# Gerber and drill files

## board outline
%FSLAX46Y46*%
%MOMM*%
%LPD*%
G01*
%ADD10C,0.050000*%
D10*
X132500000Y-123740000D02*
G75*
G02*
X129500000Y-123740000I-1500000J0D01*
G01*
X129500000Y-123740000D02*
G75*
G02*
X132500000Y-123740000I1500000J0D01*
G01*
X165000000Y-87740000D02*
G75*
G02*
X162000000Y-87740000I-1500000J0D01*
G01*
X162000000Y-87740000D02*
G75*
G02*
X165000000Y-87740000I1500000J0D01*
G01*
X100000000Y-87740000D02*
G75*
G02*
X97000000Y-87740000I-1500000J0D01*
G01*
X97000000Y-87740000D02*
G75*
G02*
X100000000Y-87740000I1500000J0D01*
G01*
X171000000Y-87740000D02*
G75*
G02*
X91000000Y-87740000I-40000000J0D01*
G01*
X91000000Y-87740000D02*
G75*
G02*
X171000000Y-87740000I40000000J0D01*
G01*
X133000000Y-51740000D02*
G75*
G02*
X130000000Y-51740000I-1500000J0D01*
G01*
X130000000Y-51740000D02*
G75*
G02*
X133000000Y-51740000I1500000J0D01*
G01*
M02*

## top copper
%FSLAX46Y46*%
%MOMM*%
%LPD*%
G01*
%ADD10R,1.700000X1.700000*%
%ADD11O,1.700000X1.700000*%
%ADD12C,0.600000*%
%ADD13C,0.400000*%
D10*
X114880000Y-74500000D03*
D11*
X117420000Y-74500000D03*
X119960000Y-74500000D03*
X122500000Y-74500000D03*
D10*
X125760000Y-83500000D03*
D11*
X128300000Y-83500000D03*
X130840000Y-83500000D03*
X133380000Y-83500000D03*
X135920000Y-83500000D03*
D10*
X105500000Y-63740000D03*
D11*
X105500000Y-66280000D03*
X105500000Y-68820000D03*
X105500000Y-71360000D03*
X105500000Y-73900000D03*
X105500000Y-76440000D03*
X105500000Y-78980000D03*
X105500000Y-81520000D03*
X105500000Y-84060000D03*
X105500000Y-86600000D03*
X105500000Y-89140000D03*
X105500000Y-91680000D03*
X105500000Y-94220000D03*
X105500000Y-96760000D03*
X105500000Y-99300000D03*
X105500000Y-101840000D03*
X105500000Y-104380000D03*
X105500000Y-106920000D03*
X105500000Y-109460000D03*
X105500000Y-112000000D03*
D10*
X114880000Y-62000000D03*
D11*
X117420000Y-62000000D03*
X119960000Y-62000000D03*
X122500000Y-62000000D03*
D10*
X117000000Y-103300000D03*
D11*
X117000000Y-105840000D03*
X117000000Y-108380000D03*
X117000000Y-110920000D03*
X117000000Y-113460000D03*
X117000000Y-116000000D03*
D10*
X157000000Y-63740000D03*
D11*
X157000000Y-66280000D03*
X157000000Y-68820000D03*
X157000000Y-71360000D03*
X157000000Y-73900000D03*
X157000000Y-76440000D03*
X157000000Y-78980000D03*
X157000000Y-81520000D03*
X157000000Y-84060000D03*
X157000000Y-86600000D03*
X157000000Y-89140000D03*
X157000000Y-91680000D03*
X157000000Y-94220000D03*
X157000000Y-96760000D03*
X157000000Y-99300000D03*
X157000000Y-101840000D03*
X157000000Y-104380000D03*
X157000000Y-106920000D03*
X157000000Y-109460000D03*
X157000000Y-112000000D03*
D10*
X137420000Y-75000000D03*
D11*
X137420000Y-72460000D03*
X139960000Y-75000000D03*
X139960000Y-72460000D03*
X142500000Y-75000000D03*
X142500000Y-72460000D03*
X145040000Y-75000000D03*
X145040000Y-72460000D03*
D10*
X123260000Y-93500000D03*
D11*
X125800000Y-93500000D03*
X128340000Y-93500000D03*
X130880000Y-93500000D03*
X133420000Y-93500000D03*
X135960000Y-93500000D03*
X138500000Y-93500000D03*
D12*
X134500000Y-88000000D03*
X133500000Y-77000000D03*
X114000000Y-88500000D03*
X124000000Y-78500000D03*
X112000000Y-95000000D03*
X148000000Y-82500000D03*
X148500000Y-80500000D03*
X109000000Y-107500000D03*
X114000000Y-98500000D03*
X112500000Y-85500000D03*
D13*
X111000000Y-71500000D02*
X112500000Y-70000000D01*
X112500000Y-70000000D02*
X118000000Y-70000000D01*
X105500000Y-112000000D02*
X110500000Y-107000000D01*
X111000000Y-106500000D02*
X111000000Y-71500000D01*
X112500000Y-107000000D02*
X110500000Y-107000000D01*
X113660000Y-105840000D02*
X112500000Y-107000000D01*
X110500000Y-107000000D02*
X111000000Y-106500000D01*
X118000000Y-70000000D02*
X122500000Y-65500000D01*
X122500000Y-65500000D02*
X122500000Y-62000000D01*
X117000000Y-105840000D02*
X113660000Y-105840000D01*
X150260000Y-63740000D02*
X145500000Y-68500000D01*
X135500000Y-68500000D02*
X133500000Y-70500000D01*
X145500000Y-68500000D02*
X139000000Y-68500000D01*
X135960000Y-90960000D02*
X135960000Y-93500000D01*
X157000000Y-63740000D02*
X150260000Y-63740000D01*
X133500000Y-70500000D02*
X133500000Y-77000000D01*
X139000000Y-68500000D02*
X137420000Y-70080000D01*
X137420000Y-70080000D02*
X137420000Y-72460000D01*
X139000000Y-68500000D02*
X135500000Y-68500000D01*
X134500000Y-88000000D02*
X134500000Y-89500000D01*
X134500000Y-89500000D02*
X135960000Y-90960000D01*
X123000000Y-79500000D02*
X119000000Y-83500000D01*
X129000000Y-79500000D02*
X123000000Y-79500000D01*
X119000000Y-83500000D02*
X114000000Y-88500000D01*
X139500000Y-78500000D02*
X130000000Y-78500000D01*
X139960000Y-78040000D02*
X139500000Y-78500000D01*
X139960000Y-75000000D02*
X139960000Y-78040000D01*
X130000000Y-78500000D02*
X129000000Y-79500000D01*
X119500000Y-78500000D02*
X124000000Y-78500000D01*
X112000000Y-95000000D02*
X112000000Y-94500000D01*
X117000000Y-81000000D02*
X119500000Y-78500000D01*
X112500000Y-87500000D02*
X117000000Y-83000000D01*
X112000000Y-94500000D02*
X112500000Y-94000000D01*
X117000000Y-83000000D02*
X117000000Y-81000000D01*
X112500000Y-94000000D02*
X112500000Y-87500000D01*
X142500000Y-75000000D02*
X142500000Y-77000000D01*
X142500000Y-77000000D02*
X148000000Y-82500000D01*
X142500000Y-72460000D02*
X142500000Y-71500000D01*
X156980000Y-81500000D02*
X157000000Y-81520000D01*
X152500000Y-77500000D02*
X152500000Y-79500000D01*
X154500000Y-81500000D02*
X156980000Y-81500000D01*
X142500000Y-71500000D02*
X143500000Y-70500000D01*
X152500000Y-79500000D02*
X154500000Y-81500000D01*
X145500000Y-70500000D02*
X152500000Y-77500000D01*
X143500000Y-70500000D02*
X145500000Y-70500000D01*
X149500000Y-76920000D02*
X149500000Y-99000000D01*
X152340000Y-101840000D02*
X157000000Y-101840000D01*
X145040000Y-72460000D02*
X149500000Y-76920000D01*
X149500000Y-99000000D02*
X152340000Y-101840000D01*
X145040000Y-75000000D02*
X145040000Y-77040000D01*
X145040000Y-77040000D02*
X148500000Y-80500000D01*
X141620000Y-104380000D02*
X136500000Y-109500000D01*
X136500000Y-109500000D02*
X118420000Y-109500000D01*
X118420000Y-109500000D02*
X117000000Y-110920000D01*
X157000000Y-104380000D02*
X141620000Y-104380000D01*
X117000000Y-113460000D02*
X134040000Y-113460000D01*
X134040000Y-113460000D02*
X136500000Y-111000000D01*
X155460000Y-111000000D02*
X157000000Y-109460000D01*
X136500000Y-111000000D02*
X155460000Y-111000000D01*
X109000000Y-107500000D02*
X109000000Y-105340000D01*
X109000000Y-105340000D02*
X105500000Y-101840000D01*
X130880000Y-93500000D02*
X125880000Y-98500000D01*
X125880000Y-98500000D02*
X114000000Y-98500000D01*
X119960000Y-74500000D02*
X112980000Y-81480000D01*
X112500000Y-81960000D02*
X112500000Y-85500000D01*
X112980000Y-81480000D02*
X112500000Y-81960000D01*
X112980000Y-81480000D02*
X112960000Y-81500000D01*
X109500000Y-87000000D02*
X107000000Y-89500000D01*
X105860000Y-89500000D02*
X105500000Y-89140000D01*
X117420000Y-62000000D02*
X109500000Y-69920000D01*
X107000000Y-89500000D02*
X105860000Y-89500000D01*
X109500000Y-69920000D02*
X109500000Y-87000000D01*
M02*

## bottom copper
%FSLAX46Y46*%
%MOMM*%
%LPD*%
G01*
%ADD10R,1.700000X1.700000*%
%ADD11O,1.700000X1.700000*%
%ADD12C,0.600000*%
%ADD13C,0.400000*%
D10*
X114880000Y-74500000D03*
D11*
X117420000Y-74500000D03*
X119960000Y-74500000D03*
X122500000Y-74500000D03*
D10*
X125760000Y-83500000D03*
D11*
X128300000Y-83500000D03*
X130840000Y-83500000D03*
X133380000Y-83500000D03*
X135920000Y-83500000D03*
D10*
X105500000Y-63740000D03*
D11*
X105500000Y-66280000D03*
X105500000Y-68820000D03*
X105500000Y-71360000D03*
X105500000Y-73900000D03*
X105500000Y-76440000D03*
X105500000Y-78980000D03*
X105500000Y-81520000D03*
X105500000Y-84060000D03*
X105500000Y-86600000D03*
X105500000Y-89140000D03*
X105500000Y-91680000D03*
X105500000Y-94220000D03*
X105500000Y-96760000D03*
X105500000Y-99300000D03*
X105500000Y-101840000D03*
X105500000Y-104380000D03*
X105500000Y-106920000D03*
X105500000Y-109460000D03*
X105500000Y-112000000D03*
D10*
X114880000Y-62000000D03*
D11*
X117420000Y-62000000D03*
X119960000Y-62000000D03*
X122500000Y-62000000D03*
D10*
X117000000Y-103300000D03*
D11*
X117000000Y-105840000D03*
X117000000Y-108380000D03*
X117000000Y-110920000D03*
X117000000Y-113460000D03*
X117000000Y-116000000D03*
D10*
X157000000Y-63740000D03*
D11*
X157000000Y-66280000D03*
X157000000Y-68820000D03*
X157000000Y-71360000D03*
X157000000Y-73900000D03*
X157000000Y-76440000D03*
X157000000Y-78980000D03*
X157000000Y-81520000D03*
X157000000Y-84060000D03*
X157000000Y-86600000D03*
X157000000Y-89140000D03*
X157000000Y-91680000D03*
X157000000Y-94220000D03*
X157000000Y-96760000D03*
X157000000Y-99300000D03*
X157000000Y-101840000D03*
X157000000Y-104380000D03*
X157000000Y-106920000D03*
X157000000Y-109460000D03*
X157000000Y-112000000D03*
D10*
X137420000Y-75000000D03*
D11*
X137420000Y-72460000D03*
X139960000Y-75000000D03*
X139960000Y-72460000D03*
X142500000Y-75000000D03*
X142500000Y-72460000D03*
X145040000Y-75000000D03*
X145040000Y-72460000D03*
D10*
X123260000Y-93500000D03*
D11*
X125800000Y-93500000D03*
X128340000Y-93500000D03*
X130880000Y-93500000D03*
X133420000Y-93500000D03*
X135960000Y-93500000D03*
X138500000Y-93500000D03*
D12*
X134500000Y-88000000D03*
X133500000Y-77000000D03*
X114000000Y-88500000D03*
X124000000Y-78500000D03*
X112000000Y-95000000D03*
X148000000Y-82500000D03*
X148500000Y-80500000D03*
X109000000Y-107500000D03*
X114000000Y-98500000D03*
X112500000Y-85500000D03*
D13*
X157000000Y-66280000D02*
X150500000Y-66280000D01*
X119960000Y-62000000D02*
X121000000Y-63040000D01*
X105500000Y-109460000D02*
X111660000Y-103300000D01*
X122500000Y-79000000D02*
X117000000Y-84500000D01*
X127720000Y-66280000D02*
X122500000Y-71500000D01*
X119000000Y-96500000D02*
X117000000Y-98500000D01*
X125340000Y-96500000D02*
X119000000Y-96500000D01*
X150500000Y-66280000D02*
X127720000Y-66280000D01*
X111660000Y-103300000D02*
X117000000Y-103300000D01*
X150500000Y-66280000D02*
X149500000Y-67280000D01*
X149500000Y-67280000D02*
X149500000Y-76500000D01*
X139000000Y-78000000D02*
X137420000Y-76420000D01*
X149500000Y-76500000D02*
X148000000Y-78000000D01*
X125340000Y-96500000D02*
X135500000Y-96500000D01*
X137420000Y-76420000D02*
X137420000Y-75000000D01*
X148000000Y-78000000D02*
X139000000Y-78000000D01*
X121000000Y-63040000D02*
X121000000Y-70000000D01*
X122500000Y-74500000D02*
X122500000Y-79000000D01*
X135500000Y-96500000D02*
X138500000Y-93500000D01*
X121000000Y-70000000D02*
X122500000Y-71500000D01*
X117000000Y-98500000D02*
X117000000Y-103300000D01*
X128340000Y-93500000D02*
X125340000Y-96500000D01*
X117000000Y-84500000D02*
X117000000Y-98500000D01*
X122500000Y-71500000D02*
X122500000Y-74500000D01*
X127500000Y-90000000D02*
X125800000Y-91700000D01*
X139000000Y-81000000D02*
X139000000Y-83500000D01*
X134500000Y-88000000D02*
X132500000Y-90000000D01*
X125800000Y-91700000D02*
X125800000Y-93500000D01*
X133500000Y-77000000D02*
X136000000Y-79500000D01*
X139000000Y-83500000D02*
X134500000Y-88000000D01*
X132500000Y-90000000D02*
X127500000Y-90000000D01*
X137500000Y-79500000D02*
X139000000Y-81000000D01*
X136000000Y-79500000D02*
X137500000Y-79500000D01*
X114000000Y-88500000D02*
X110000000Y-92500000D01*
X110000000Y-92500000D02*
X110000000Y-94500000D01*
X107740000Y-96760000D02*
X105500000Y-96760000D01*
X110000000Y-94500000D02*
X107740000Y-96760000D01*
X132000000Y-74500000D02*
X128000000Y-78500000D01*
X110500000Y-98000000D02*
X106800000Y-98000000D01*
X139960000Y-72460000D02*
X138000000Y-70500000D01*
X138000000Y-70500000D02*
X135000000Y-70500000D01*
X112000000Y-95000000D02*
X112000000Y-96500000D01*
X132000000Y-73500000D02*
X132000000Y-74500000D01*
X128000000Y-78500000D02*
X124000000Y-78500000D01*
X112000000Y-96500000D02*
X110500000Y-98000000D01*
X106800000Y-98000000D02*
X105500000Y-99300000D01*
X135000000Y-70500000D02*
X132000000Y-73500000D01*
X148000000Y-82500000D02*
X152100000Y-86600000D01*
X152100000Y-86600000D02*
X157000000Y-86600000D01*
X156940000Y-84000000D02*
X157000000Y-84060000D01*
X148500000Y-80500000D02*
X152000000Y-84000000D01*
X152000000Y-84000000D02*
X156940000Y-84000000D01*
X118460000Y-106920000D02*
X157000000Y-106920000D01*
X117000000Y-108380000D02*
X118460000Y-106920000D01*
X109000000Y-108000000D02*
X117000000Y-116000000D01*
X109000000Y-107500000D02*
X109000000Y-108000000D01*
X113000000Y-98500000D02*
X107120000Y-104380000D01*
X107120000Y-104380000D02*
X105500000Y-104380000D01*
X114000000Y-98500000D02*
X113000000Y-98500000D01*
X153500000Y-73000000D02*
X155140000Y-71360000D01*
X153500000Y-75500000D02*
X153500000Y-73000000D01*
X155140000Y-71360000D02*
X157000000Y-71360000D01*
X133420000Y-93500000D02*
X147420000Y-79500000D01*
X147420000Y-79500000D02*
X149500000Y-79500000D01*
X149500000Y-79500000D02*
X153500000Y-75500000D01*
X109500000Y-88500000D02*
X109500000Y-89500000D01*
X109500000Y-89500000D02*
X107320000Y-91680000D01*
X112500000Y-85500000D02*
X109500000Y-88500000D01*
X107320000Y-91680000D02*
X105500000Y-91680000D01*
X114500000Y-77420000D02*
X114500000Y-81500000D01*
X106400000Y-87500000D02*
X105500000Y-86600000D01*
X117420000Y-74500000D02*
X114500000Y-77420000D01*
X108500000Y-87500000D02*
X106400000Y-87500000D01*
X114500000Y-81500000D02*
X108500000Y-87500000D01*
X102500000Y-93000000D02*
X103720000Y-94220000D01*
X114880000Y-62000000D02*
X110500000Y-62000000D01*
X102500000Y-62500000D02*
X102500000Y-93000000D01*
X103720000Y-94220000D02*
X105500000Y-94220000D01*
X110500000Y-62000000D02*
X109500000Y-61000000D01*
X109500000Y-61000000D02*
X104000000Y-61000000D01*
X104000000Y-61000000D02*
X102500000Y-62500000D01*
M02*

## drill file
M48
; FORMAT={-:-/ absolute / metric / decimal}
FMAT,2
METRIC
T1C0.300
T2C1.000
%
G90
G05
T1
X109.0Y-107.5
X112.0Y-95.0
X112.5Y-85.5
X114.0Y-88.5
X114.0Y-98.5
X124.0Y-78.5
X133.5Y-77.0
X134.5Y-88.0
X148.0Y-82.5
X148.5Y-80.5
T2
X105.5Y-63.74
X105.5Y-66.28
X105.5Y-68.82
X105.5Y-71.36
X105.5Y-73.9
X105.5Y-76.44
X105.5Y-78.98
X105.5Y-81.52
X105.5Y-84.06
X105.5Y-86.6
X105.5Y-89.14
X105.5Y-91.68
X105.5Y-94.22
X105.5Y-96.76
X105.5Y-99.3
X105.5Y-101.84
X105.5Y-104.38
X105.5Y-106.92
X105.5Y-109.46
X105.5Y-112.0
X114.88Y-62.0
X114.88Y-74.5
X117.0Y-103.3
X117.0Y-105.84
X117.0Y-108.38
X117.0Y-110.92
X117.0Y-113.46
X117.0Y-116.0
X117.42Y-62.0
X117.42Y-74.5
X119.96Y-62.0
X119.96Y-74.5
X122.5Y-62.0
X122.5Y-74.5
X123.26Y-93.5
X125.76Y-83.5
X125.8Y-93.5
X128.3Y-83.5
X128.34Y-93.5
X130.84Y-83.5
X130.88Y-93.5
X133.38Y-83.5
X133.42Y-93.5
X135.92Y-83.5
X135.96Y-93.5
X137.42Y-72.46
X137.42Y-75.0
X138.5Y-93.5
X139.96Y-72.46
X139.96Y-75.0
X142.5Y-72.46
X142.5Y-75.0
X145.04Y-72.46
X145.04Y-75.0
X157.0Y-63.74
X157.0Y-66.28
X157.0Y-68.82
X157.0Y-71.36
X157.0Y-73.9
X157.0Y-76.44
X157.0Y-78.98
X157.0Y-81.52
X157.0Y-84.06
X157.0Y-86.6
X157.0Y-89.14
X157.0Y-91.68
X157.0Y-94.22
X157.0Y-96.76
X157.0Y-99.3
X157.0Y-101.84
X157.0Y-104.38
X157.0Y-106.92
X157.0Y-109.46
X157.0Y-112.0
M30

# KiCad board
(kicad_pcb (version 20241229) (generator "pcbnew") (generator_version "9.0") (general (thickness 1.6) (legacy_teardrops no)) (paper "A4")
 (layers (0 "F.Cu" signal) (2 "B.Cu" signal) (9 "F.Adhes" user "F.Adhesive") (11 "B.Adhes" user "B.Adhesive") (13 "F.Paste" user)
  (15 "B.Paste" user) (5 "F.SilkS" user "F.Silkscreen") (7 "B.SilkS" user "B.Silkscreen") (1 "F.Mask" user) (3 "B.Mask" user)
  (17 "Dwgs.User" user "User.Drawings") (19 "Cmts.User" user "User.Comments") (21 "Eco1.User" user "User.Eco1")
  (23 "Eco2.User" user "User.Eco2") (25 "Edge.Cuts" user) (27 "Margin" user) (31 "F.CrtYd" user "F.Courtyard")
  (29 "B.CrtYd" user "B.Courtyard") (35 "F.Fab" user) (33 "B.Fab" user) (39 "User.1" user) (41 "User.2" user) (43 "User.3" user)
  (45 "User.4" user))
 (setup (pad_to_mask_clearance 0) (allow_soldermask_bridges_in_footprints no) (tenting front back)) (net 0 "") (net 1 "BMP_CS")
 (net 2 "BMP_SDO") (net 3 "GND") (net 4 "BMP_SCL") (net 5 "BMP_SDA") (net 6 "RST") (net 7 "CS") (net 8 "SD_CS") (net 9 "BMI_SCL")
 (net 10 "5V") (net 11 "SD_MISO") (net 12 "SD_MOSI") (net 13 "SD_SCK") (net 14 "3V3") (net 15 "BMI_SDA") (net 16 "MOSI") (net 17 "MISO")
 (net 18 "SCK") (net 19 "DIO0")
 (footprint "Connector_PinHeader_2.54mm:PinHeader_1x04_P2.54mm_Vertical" (layer "F.Cu") (at 114.88 74.5 90)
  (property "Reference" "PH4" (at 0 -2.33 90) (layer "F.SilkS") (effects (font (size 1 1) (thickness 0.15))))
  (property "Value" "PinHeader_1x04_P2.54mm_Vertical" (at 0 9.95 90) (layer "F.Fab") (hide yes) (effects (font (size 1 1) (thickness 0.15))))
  (pad "1" thru_hole rect (at 0 0 90) (size 1.7 1.7) (drill 1) (layers "*.Cu" "*.Mask") (remove_unused_layers no))
  (pad "2" thru_hole oval (at 0 2.54 90) (size 1.7 1.7) (drill 1) (layers "*.Cu" "*.Mask") (remove_unused_layers no) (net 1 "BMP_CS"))
  (pad "3" thru_hole oval (at 0 5.08 90) (size 1.7 1.7) (drill 1) (layers "*.Cu" "*.Mask") (remove_unused_layers no) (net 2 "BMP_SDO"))
  (pad "4" thru_hole oval (at 0 7.62 90) (size 1.7 1.7) (drill 1) (layers "*.Cu" "*.Mask") (remove_unused_layers no) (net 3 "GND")))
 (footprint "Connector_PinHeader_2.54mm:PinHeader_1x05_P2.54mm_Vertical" (layer "F.Cu") (at 125.76 83.5 90)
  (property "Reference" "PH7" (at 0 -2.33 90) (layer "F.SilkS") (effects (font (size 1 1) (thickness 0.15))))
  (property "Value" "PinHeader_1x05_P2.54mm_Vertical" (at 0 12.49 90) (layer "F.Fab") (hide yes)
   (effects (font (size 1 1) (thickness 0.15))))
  (pad "1" thru_hole rect (at 0 0 90) (size 1.7 1.7) (drill 1) (layers "*.Cu" "*.Mask") (remove_unused_layers no))
  (pad "2" thru_hole oval (at 0 2.54 90) (size 1.7 1.7) (drill 1) (layers "*.Cu" "*.Mask") (remove_unused_layers no))
  (pad "3" thru_hole oval (at 0 5.08 90) (size 1.7 1.7) (drill 1) (layers "*.Cu" "*.Mask") (remove_unused_layers no))
  (pad "4" thru_hole oval (at 0 7.62 90) (size 1.7 1.7) (drill 1) (layers "*.Cu" "*.Mask") (remove_unused_layers no))
  (pad "5" thru_hole oval (at 0 10.16 90) (size 1.7 1.7) (drill 1) (layers "*.Cu" "*.Mask") (remove_unused_layers no)))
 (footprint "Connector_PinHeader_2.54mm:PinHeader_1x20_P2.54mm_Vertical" (layer "F.Cu") (at 105.5 63.74)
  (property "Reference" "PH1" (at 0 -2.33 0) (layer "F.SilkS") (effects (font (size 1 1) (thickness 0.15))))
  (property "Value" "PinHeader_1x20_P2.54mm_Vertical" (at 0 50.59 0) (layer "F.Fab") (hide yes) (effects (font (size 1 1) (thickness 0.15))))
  (pad "1" thru_hole rect (at 0 0) (size 1.7 1.7) (drill 1) (layers "*.Cu" "*.Mask") (remove_unused_layers no))
  (pad "2" thru_hole oval (at 0 2.54) (size 1.7 1.7) (drill 1) (layers "*.Cu" "*.Mask") (remove_unused_layers no))
  (pad "3" thru_hole oval (at 0 5.08) (size 1.7 1.7) (drill 1) (layers "*.Cu" "*.Mask") (remove_unused_layers no))
  (pad "4" thru_hole oval (at 0 7.62) (size 1.7 1.7) (drill 1) (layers "*.Cu" "*.Mask") (remove_unused_layers no))
  (pad "5" thru_hole oval (at 0 10.16) (size 1.7 1.7) (drill 1) (layers "*.Cu" "*.Mask") (remove_unused_layers no))
  (pad "6" thru_hole oval (at 0 12.7) (size 1.7 1.7) (drill 1) (layers "*.Cu" "*.Mask") (remove_unused_layers no))
  (pad "7" thru_hole oval (at 0 15.24) (size 1.7 1.7) (drill 1) (layers "*.Cu" "*.Mask") (remove_unused_layers no))
  (pad "8" thru_hole oval (at 0 17.78) (size 1.7 1.7) (drill 1) (layers "*.Cu" "*.Mask") (remove_unused_layers no))
  (pad "9" thru_hole oval (at 0 20.32) (size 1.7 1.7) (drill 1) (layers "*.Cu" "*.Mask") (remove_unused_layers no))
  (pad "10" thru_hole oval (at 0 22.86) (size 1.7 1.7) (drill 1) (layers "*.Cu" "*.Mask") (remove_unused_layers no) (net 1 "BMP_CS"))
  (pad "11" thru_hole oval (at 0 25.4) (size 1.7 1.7) (drill 1) (layers "*.Cu" "*.Mask") (remove_unused_layers no) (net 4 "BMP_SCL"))
  (pad "12" thru_hole oval (at 0 27.94) (size 1.7 1.7) (drill 1) (layers "*.Cu" "*.Mask") (remove_unused_layers no) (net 2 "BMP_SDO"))
  (pad "13" thru_hole oval (at 0 30.48) (size 1.7 1.7) (drill 1) (layers "*.Cu" "*.Mask") (remove_unused_layers no) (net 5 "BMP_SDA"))
  (pad "14" thru_hole oval (at 0 33.02) (size 1.7 1.7) (drill 1) (layers "*.Cu" "*.Mask") (remove_unused_layers no) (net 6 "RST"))
  (pad "15" thru_hole oval (at 0 35.56) (size 1.7 1.7) (drill 1) (layers "*.Cu" "*.Mask") (remove_unused_layers no) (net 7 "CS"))
  (pad "16" thru_hole oval (at 0 38.1) (size 1.7 1.7) (drill 1) (layers "*.Cu" "*.Mask") (remove_unused_layers no) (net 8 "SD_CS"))
  (pad "17" thru_hole oval (at 0 40.64) (size 1.7 1.7) (drill 1) (layers "*.Cu" "*.Mask") (remove_unused_layers no) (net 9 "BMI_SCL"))
  (pad "18" thru_hole oval (at 0 43.18) (size 1.7 1.7) (drill 1) (layers "*.Cu" "*.Mask") (remove_unused_layers no))
  (pad "19" thru_hole oval (at 0 45.72) (size 1.7 1.7) (drill 1) (layers "*.Cu" "*.Mask") (remove_unused_layers no) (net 3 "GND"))
  (pad "20" thru_hole oval (at 0 48.26) (size 1.7 1.7) (drill 1) (layers "*.Cu" "*.Mask") (remove_unused_layers no) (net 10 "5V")))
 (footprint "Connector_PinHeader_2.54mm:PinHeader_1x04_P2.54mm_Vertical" (layer "F.Cu") (at 114.88 62 90)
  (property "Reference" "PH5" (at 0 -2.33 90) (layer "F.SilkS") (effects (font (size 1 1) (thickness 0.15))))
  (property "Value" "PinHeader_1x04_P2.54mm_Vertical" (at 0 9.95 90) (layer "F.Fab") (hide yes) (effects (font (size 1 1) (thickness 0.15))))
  (pad "1" thru_hole rect (at 0 0 90) (size 1.7 1.7) (drill 1) (layers "*.Cu" "*.Mask") (remove_unused_layers no) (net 5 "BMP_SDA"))
  (pad "2" thru_hole oval (at 0 2.54 90) (size 1.7 1.7) (drill 1) (layers "*.Cu" "*.Mask") (remove_unused_layers no) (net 4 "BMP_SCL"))
  (pad "3" thru_hole oval (at 0 5.08 90) (size 1.7 1.7) (drill 1) (layers "*.Cu" "*.Mask") (remove_unused_layers no) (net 3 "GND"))
  (pad "4" thru_hole oval (at 0 7.62 90) (size 1.7 1.7) (drill 1) (layers "*.Cu" "*.Mask") (remove_unused_layers no) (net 10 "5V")))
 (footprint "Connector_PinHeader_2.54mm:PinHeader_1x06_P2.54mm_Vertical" (layer "F.Cu") (at 117 103.3)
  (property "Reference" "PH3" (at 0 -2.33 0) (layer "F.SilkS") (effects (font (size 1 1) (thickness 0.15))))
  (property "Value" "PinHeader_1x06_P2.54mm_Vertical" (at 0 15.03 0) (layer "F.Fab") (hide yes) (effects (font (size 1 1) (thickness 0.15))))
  (pad "1" thru_hole rect (at 0 0) (size 1.7 1.7) (drill 1) (layers "*.Cu" "*.Mask") (remove_unused_layers no) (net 3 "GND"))
  (pad "2" thru_hole oval (at 0 2.54) (size 1.7 1.7) (drill 1) (layers "*.Cu" "*.Mask") (remove_unused_layers no) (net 10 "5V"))
  (pad "3" thru_hole oval (at 0 5.08) (size 1.7 1.7) (drill 1) (layers "*.Cu" "*.Mask") (remove_unused_layers no) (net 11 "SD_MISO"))
  (pad "4" thru_hole oval (at 0 7.62) (size 1.7 1.7) (drill 1) (layers "*.Cu" "*.Mask") (remove_unused_layers no) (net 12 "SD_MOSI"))
  (pad "5" thru_hole oval (at 0 10.16) (size 1.7 1.7) (drill 1) (layers "*.Cu" "*.Mask") (remove_unused_layers no) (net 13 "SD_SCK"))
  (pad "6" thru_hole oval (at 0 12.7) (size 1.7 1.7) (drill 1) (layers "*.Cu" "*.Mask") (remove_unused_layers no) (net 8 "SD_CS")))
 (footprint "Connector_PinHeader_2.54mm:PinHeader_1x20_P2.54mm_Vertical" (layer "F.Cu") (at 157 63.74)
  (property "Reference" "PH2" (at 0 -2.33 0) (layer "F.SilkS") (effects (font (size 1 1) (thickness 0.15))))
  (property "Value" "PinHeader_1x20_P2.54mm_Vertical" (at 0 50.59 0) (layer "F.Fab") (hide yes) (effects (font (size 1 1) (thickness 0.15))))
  (pad "1" thru_hole rect (at 0 0) (size 1.7 1.7) (drill 1) (layers "*.Cu" "*.Mask") (remove_unused_layers no) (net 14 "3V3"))
  (pad "2" thru_hole oval (at 0 2.54) (size 1.7 1.7) (drill 1) (layers "*.Cu" "*.Mask") (remove_unused_layers no) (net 3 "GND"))
  (pad "3" thru_hole oval (at 0 5.08) (size 1.7 1.7) (drill 1) (layers "*.Cu" "*.Mask") (remove_unused_layers no))
  (pad "4" thru_hole oval (at 0 7.62) (size 1.7 1.7) (drill 1) (layers "*.Cu" "*.Mask") (remove_unused_layers no) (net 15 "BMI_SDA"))
  (pad "5" thru_hole oval (at 0 10.16) (size 1.7 1.7) (drill 1) (layers "*.Cu" "*.Mask") (remove_unused_layers no))
  (pad "6" thru_hole oval (at 0 12.7) (size 1.7 1.7) (drill 1) (layers "*.Cu" "*.Mask") (remove_unused_layers no))
  (pad "7" thru_hole oval (at 0 15.24) (size 1.7 1.7) (drill 1) (layers "*.Cu" "*.Mask") (remove_unused_layers no))
  (pad "8" thru_hole oval (at 0 17.78) (size 1.7 1.7) (drill 1) (layers "*.Cu" "*.Mask") (remove_unused_layers no) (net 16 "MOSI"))
  (pad "9" thru_hole oval (at 0 20.32) (size 1.7 1.7) (drill 1) (layers "*.Cu" "*.Mask") (remove_unused_layers no) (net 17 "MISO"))
  (pad "10" thru_hole oval (at 0 22.86) (size 1.7 1.7) (drill 1) (layers "*.Cu" "*.Mask") (remove_unused_layers no) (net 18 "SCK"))
  (pad "11" thru_hole oval (at 0 25.4) (size 1.7 1.7) (drill 1) (layers "*.Cu" "*.Mask") (remove_unused_layers no))
  (pad "12" thru_hole oval (at 0 27.94) (size 1.7 1.7) (drill 1) (layers "*.Cu" "*.Mask") (remove_unused_layers no))
  (pad "13" thru_hole oval (at 0 30.48) (size 1.7 1.7) (drill 1) (layers "*.Cu" "*.Mask") (remove_unused_layers no))
  (pad "14" thru_hole oval (at 0 33.02) (size 1.7 1.7) (drill 1) (layers "*.Cu" "*.Mask") (remove_unused_layers no))
  (pad "15" thru_hole oval (at 0 35.56) (size 1.7 1.7) (drill 1) (layers "*.Cu" "*.Mask") (remove_unused_layers no))
  (pad "16" thru_hole oval (at 0 38.1) (size 1.7 1.7) (drill 1) (layers "*.Cu" "*.Mask") (remove_unused_layers no) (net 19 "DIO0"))
  (pad "17" thru_hole oval (at 0 40.64) (size 1.7 1.7) (drill 1) (layers "*.Cu" "*.Mask") (remove_unused_layers no) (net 12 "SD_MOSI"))
  (pad "18" thru_hole oval (at 0 43.18) (size 1.7 1.7) (drill 1) (layers "*.Cu" "*.Mask") (remove_unused_layers no) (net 11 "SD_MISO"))
  (pad "19" thru_hole oval (at 0 45.72) (size 1.7 1.7) (drill 1) (layers "*.Cu" "*.Mask") (remove_unused_layers no) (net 13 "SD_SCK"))
  (pad "20" thru_hole oval (at 0 48.26) (size 1.7 1.7) (drill 1) (layers "*.Cu" "*.Mask") (remove_unused_layers no)))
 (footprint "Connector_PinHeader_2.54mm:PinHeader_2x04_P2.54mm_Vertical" (layer "F.Cu") (at 137.42 75 90)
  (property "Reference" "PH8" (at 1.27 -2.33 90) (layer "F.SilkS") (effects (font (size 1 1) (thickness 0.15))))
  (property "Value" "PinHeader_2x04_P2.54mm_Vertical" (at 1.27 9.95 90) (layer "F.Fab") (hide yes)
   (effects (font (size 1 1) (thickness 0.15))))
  (pad "1" thru_hole rect (at 0 0 90) (size 1.7 1.7) (drill 1) (layers "*.Cu" "*.Mask") (remove_unused_layers no) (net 3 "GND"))
  (pad "2" thru_hole oval (at 2.54 0 90) (size 1.7 1.7) (drill 1) (layers "*.Cu" "*.Mask") (remove_unused_layers no) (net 14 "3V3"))
  (pad "3" thru_hole oval (at 0 2.54 90) (size 1.7 1.7) (drill 1) (layers "*.Cu" "*.Mask") (remove_unused_layers no) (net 6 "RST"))
  (pad "4" thru_hole oval (at 2.54 2.54 90) (size 1.7 1.7) (drill 1) (layers "*.Cu" "*.Mask") (remove_unused_layers no) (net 7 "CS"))
  (pad "5" thru_hole oval (at 0 5.08 90) (size 1.7 1.7) (drill 1) (layers "*.Cu" "*.Mask") (remove_unused_layers no) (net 18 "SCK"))
  (pad "6" thru_hole oval (at 2.54 5.08 90) (size 1.7 1.7) (drill 1) (layers "*.Cu" "*.Mask") (remove_unused_layers no) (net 16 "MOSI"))
  (pad "7" thru_hole oval (at 0 7.62 90) (size 1.7 1.7) (drill 1) (layers "*.Cu" "*.Mask") (remove_unused_layers no) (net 17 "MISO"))
  (pad "8" thru_hole oval (at 2.54 7.62 90) (size 1.7 1.7) (drill 1) (layers "*.Cu" "*.Mask") (remove_unused_layers no) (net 19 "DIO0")))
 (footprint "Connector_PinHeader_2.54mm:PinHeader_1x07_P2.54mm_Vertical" (layer "F.Cu") (at 123.26 93.5 90)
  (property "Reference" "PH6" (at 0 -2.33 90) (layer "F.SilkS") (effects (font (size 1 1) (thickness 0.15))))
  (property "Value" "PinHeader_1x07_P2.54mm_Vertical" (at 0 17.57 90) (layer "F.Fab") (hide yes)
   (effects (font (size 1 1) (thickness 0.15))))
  (pad "1" thru_hole rect (at 0 0 90) (size 1.7 1.7) (drill 1) (layers "*.Cu" "*.Mask") (remove_unused_layers no))
  (pad "2" thru_hole oval (at 0 2.54 90) (size 1.7 1.7) (drill 1) (layers "*.Cu" "*.Mask") (remove_unused_layers no) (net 14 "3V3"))
  (pad "3" thru_hole oval (at 0 5.08 90) (size 1.7 1.7) (drill 1) (layers "*.Cu" "*.Mask") (remove_unused_layers no) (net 3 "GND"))
  (pad "4" thru_hole oval (at 0 7.62 90) (size 1.7 1.7) (drill 1) (layers "*.Cu" "*.Mask") (remove_unused_layers no) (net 9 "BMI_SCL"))
  (pad "5" thru_hole oval (at 0 10.16 90) (size 1.7 1.7) (drill 1) (layers "*.Cu" "*.Mask") (remove_unused_layers no) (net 15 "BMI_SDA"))
  (pad "6" thru_hole oval (at 0 12.7 90) (size 1.7 1.7) (drill 1) (layers "*.Cu" "*.Mask") (remove_unused_layers no) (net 14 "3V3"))
  (pad "7" thru_hole oval (at 0 15.24 90) (size 1.7 1.7) (drill 1) (layers "*.Cu" "*.Mask") (remove_unused_layers no) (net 3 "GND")))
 (gr_circle (center 131 123.74) (end 132.5 123.74) (stroke (width 0.05) (type default)) (fill no) (layer "Edge.Cuts"))
 (gr_circle (center 163.5 87.74) (end 165 87.74) (stroke (width 0.05) (type default)) (fill no) (layer "Edge.Cuts"))
 (gr_circle (center 98.5 87.74) (end 100 87.74) (stroke (width 0.05) (type default)) (fill no) (layer "Edge.Cuts"))
 (gr_circle (center 131 87.74) (end 171 87.74) (stroke (width 0.05) (type default)) (fill no) (layer "Edge.Cuts"))
 (gr_circle (center 131.5 51.74) (end 133 51.74) (stroke (width 0.05) (type default)) (fill no) (layer "Edge.Cuts"))
 (segment (start 157 66.28) (end 150.5 66.28) (width 0.4) (layer "B.Cu") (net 3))
 (segment (start 119.96 62) (end 121 63.04) (width 0.4) (layer "B.Cu") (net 3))
 (segment (start 105.5 109.46) (end 111.66 103.3) (width 0.4) (layer "B.Cu") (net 3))
 (segment (start 122.5 79) (end 117 84.5) (width 0.4) (layer "B.Cu") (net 3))
 (segment (start 127.72 66.28) (end 122.5 71.5) (width 0.4) (layer "B.Cu") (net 3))
 (segment (start 119 96.5) (end 117 98.5) (width 0.4) (layer "B.Cu") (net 3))
 (segment (start 125.34 96.5) (end 119 96.5) (width 0.4) (layer "B.Cu") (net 3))
 (segment (start 150.5 66.28) (end 127.72 66.28) (width 0.4) (layer "B.Cu") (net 3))
 (segment (start 111.66 103.3) (end 117 103.3) (width 0.4) (layer "B.Cu") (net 3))
 (segment (start 150.5 66.28) (end 149.5 67.28) (width 0.4) (layer "B.Cu") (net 3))
 (segment (start 149.5 67.28) (end 149.5 76.5) (width 0.4) (layer "B.Cu") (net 3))
 (segment (start 139 78) (end 137.42 76.42) (width 0.4) (layer "B.Cu") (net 3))
 (segment (start 149.5 76.5) (end 148 78) (width 0.4) (layer "B.Cu") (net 3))
 (segment (start 125.34 96.5) (end 135.5 96.5) (width 0.4) (layer "B.Cu") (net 3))
 (segment (start 137.42 76.42) (end 137.42 75) (width 0.4) (layer "B.Cu") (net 3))
 (segment (start 148 78) (end 139 78) (width 0.4) (layer "B.Cu") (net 3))
 (segment (start 121 63.04) (end 121 70) (width 0.4) (layer "B.Cu") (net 3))
 (segment (start 122.5 74.5) (end 122.5 79) (width 0.4) (layer "B.Cu") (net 3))
 (segment (start 135.5 96.5) (end 138.5 93.5) (width 0.4) (layer "B.Cu") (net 3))
 (segment (start 121 70) (end 122.5 71.5) (width 0.4) (layer "B.Cu") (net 3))
 (segment (start 117 98.5) (end 117 103.3) (width 0.4) (layer "B.Cu") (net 3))
 (segment (start 128.34 93.5) (end 125.34 96.5) (width 0.4) (layer "B.Cu") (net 3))
 (segment (start 117 84.5) (end 117 98.5) (width 0.4) (layer "B.Cu") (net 3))
 (segment (start 122.5 71.5) (end 122.5 74.5) (width 0.4) (layer "B.Cu") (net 3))
 (segment (start 111 71.5) (end 112.5 70) (width 0.4) (layer "F.Cu") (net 10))
 (segment (start 112.5 70) (end 118 70) (width 0.4) (layer "F.Cu") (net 10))
 (segment (start 105.5 112) (end 110.5 107) (width 0.4) (layer "F.Cu") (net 10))
 (segment (start 111 106.5) (end 111 71.5) (width 0.4) (layer "F.Cu") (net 10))
 (segment (start 112.5 107) (end 110.5 107) (width 0.4) (layer "F.Cu") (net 10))
 (segment (start 113.66 105.84) (end 112.5 107) (width 0.4) (layer "F.Cu") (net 10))
 (segment (start 110.5 107) (end 111 106.5) (width 0.4) (layer "F.Cu") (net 10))
 (segment (start 118 70) (end 122.5 65.5) (width 0.4) (layer "F.Cu") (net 10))
 (segment (start 122.5 65.5) (end 122.5 62) (width 0.4) (layer "F.Cu") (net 10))
 (segment (start 117 105.84) (end 113.66 105.84) (width 0.4) (layer "F.Cu") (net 10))
 (segment (start 150.26 63.74) (end 145.5 68.5) (width 0.4) (layer "F.Cu") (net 14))
 (segment (start 135.5 68.5) (end 133.5 70.5) (width 0.4) (layer "F.Cu") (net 14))
 (segment (start 145.5 68.5) (end 139 68.5) (width 0.4) (layer "F.Cu") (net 14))
 (segment (start 135.96 90.96) (end 135.96 93.5) (width 0.4) (layer "F.Cu") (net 14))
 (segment (start 157 63.74) (end 150.26 63.74) (width 0.4) (layer "F.Cu") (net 14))
 (segment (start 133.5 70.5) (end 133.5 77) (width 0.4) (layer "F.Cu") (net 14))
 (segment (start 139 68.5) (end 137.42 70.08) (width 0.4) (layer "F.Cu") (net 14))
 (segment (start 137.42 70.08) (end 137.42 72.46) (width 0.4) (layer "F.Cu") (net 14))
 (segment (start 139 68.5) (end 135.5 68.5) (width 0.4) (layer "F.Cu") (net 14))
 (segment (start 134.5 88) (end 134.5 89.5) (width 0.4) (layer "F.Cu") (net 14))
 (segment (start 134.5 89.5) (end 135.96 90.96) (width 0.4) (layer "F.Cu") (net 14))
 (via (at 134.5 88) (size 0.6) (drill 0.3) (layers "F.Cu" "B.Cu") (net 14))
 (via (at 133.5 77) (size 0.6) (drill 0.3) (layers "F.Cu" "B.Cu") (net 14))
 (segment (start 127.5 90) (end 125.8 91.7) (width 0.4) (layer "B.Cu") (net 14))
 (segment (start 139 81) (end 139 83.5) (width 0.4) (layer "B.Cu") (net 14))
 (segment (start 134.5 88) (end 132.5 90) (width 0.4) (layer "B.Cu") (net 14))
 (segment (start 125.8 91.7) (end 125.8 93.5) (width 0.4) (layer "B.Cu") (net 14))
 (segment (start 133.5 77) (end 136 79.5) (width 0.4) (layer "B.Cu") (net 14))
 (segment (start 139 83.5) (end 134.5 88) (width 0.4) (layer "B.Cu") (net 14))
 (segment (start 132.5 90) (end 127.5 90) (width 0.4) (layer "B.Cu") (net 14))
 (segment (start 137.5 79.5) (end 139 81) (width 0.4) (layer "B.Cu") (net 14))
 (segment (start 136 79.5) (end 137.5 79.5) (width 0.4) (layer "B.Cu") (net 14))
 (segment (start 123 79.5) (end 119 83.5) (width 0.4) (layer "F.Cu") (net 6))
 (segment (start 129 79.5) (end 123 79.5) (width 0.4) (layer "F.Cu") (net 6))
 (segment (start 119 83.5) (end 114 88.5) (width 0.4) (layer "F.Cu") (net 6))
 (segment (start 139.5 78.5) (end 130 78.5) (width 0.4) (layer "F.Cu") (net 6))
 (segment (start 139.96 78.04) (end 139.5 78.5) (width 0.4) (layer "F.Cu") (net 6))
 (segment (start 139.96 75) (end 139.96 78.04) (width 0.4) (layer "F.Cu") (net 6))
 (segment (start 130 78.5) (end 129 79.5) (width 0.4) (layer "F.Cu") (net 6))
 (via (at 114 88.5) (size 0.6) (drill 0.3) (layers "F.Cu" "B.Cu") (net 6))
 (segment (start 114 88.5) (end 110 92.5) (width 0.4) (layer "B.Cu") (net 6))
 (segment (start 110 92.5) (end 110 94.5) (width 0.4) (layer "B.Cu") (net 6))
 (segment (start 107.74 96.76) (end 105.5 96.76) (width 0.4) (layer "B.Cu") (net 6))
 (segment (start 110 94.5) (end 107.74 96.76) (width 0.4) (layer "B.Cu") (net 6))
 (segment (start 119.5 78.5) (end 124 78.5) (width 0.4) (layer "F.Cu") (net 7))
 (segment (start 112 95) (end 112 94.5) (width 0.4) (layer "F.Cu") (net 7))
 (segment (start 117 81) (end 119.5 78.5) (width 0.4) (layer "F.Cu") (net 7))
 (segment (start 112.5 87.5) (end 117 83) (width 0.4) (layer "F.Cu") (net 7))
 (segment (start 112 94.5) (end 112.5 94) (width 0.4) (layer "F.Cu") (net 7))
 (segment (start 117 83) (end 117 81) (width 0.4) (layer "F.Cu") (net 7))
 (segment (start 112.5 94) (end 112.5 87.5) (width 0.4) (layer "F.Cu") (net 7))
 (via (at 124 78.5) (size 0.6) (drill 0.3) (layers "F.Cu" "B.Cu") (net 7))
 (via (at 112 95) (size 0.6) (drill 0.3) (layers "F.Cu" "B.Cu") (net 7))
 (segment (start 132 74.5) (end 128 78.5) (width 0.4) (layer "B.Cu") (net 7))
 (segment (start 110.5 98) (end 106.8 98) (width 0.4) (layer "B.Cu") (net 7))
 (segment (start 139.96 72.46) (end 138 70.5) (width 0.4) (layer "B.Cu") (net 7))
 (segment (start 138 70.5) (end 135 70.5) (width 0.4) (layer "B.Cu") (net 7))
 (segment (start 112 95) (end 112 96.5) (width 0.4) (layer "B.Cu") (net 7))
 (segment (start 132 73.5) (end 132 74.5) (width 0.4) (layer "B.Cu") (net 7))
 (segment (start 128 78.5) (end 124 78.5) (width 0.4) (layer "B.Cu") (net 7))
 (segment (start 112 96.5) (end 110.5 98) (width 0.4) (layer "B.Cu") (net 7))
 (segment (start 106.8 98) (end 105.5 99.3) (width 0.4) (layer "B.Cu") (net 7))
 (segment (start 135 70.5) (end 132 73.5) (width 0.4) (layer "B.Cu") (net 7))
 (segment (start 142.5 75) (end 142.5 77) (width 0.4) (layer "F.Cu") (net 18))
 (segment (start 142.5 77) (end 148 82.5) (width 0.4) (layer "F.Cu") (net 18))
 (via (at 148 82.5) (size 0.6) (drill 0.3) (layers "F.Cu" "B.Cu") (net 18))
 (segment (start 148 82.5) (end 152.1 86.6) (width 0.4) (layer "B.Cu") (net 18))
 (segment (start 152.1 86.6) (end 157 86.6) (width 0.4) (layer "B.Cu") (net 18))
 (segment (start 142.5 72.46) (end 142.5 71.5) (width 0.4) (layer "F.Cu") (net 16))
 (segment (start 156.98 81.5) (end 157 81.52) (width 0.4) (layer "F.Cu") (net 16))
 (segment (start 152.5 77.5) (end 152.5 79.5) (width 0.4) (layer "F.Cu") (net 16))
 (segment (start 154.5 81.5) (end 156.98 81.5) (width 0.4) (layer "F.Cu") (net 16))
 (segment (start 142.5 71.5) (end 143.5 70.5) (width 0.4) (layer "F.Cu") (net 16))
 (segment (start 152.5 79.5) (end 154.5 81.5) (width 0.4) (layer "F.Cu") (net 16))
 (segment (start 145.5 70.5) (end 152.5 77.5) (width 0.4) (layer "F.Cu") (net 16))
 (segment (start 143.5 70.5) (end 145.5 70.5) (width 0.4) (layer "F.Cu") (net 16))
 (segment (start 149.5 76.92) (end 149.5 99) (width 0.4) (layer "F.Cu") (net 19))
 (segment (start 152.34 101.84) (end 157 101.84) (width 0.4) (layer "F.Cu") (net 19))
 (segment (start 145.04 72.46) (end 149.5 76.92) (width 0.4) (layer "F.Cu") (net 19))
 (segment (start 149.5 99) (end 152.34 101.84) (width 0.4) (layer "F.Cu") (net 19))
 (segment (start 145.04 75) (end 145.04 77.04) (width 0.4) (layer "F.Cu") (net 17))
 (segment (start 145.04 77.04) (end 148.5 80.5) (width 0.4) (layer "F.Cu") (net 17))
 (via (at 148.5 80.5) (size 0.6) (drill 0.3) (layers "F.Cu" "B.Cu") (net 17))
 (segment (start 156.94 84) (end 157 84.06) (width 0.4) (layer "B.Cu") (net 17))
 (segment (start 148.5 80.5) (end 152 84) (width 0.4) (layer "B.Cu") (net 17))
 (segment (start 152 84) (end 156.94 84) (width 0.4) (layer "B.Cu") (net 17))
 (segment (start 141.62 104.38) (end 136.5 109.5) (width 0.4) (layer "F.Cu") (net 12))
 (segment (start 136.5 109.5) (end 118.42 109.5) (width 0.4) (layer "F.Cu") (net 12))
 (segment (start 118.42 109.5) (end 117 110.92) (width 0.4) (layer "F.Cu") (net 12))
 (segment (start 157 104.38) (end 141.62 104.38) (width 0.4) (layer "F.Cu") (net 12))
 (segment (start 118.46 106.92) (end 157 106.92) (width 0.4) (layer "B.Cu") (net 11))
 (segment (start 117 108.38) (end 118.46 106.92) (width 0.4) (layer "B.Cu") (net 11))
 (segment (start 117 113.46) (end 134.04 113.46) (width 0.4) (layer "F.Cu") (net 13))
 (segment (start 134.04 113.46) (end 136.5 111) (width 0.4) (layer "F.Cu") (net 13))
 (segment (start 155.46 111) (end 157 109.46) (width 0.4) (layer "F.Cu") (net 13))
 (segment (start 136.5 111) (end 155.46 111) (width 0.4) (layer "F.Cu") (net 13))
 (segment (start 109 107.5) (end 109 105.34) (width 0.4) (layer "F.Cu") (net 8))
 (segment (start 109 105.34) (end 105.5 101.84) (width 0.4) (layer "F.Cu") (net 8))
 (via (at 109 107.5) (size 0.6) (drill 0.3) (layers "F.Cu" "B.Cu") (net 8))
 (segment (start 109 108) (end 117 116) (width 0.4) (layer "B.Cu") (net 8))
 (segment (start 109 107.5) (end 109 108) (width 0.4) (layer "B.Cu") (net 8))
 (segment (start 130.88 93.5) (end 125.88 98.5) (width 0.4) (layer "F.Cu") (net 9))
 (segment (start 125.88 98.5) (end 114 98.5) (width 0.4) (layer "F.Cu") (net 9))
 (via (at 114 98.5) (size 0.6) (drill 0.3) (layers "F.Cu" "B.Cu") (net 9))
 (segment (start 113 98.5) (end 107.12 104.38) (width 0.4) (layer "B.Cu") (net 9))
 (segment (start 107.12 104.38) (end 105.5 104.38) (width 0.4) (layer "B.Cu") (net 9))
 (segment (start 114 98.5) (end 113 98.5) (width 0.4) (layer "B.Cu") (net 9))
 (segment (start 153.5 73) (end 155.14 71.36) (width 0.4) (layer "B.Cu") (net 15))
 (segment (start 153.5 75.5) (end 153.5 73) (width 0.4) (layer "B.Cu") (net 15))
 (segment (start 155.14 71.36) (end 157 71.36) (width 0.4) (layer "B.Cu") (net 15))
 (segment (start 133.42 93.5) (end 147.42 79.5) (width 0.4) (layer "B.Cu") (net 15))
 (segment (start 147.42 79.5) (end 149.5 79.5) (width 0.4) (layer "B.Cu") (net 15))
 (segment (start 149.5 79.5) (end 153.5 75.5) (width 0.4) (layer "B.Cu") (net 15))
 (segment (start 119.96 74.5) (end 112.98 81.48) (width 0.4) (layer "F.Cu") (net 2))
 (segment (start 112.5 81.96) (end 112.5 85.5) (width 0.4) (layer "F.Cu") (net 2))
 (segment (start 112.98 81.48) (end 112.5 81.96) (width 0.4) (layer "F.Cu") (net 2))
 (segment (start 112.98 81.48) (end 112.96 81.5) (width 0.4) (layer "F.Cu") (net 2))
 (via (at 112.5 85.5) (size 0.6) (drill 0.3) (layers "F.Cu" "B.Cu") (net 2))
 (segment (start 109.5 88.5) (end 109.5 89.5) (width 0.4) (layer "B.Cu") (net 2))
 (segment (start 109.5 89.5) (end 107.32 91.68) (width 0.4) (layer "B.Cu") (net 2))
 (segment (start 112.5 85.5) (end 109.5 88.5) (width 0.4) (layer "B.Cu") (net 2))
 (segment (start 107.32 91.68) (end 105.5 91.68) (width 0.4) (layer "B.Cu") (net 2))
 (segment (start 114.5 77.42) (end 114.5 81.5) (width 0.4) (layer "B.Cu") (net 1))
 (segment (start 106.4 87.5) (end 105.5 86.6) (width 0.4) (layer "B.Cu") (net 1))
 (segment (start 117.42 74.5) (end 114.5 77.42) (width 0.4) (layer "B.Cu") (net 1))
 (segment (start 108.5 87.5) (end 106.4 87.5) (width 0.4) (layer "B.Cu") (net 1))
 (segment (start 114.5 81.5) (end 108.5 87.5) (width 0.4) (layer "B.Cu") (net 1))
 (segment (start 109.5 87) (end 107 89.5) (width 0.4) (layer "F.Cu") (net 4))
 (segment (start 105.86 89.5) (end 105.5 89.14) (width 0.4) (layer "F.Cu") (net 4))
 (segment (start 117.42 62) (end 109.5 69.92) (width 0.4) (layer "F.Cu") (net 4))
 (segment (start 107 89.5) (end 105.86 89.5) (width 0.4) (layer "F.Cu") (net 4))
 (segment (start 109.5 69.92) (end 109.5 87) (width 0.4) (layer "F.Cu") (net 4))
 (segment (start 102.5 93) (end 103.72 94.22) (width 0.4) (layer "B.Cu") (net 5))
 (segment (start 114.88 62) (end 110.5 62) (width 0.4) (layer "B.Cu") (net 5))
 (segment (start 102.5 62.5) (end 102.5 93) (width 0.4) (layer "B.Cu") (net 5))
 (segment (start 103.72 94.22) (end 105.5 94.22) (width 0.4) (layer "B.Cu") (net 5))
 (segment (start 110.5 62) (end 109.5 61) (width 0.4) (layer "B.Cu") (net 5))
 (segment (start 109.5 61) (end 104 61) (width 0.4) (layer "B.Cu") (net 5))
 (segment (start 104 61) (end 102.5 62.5) (width 0.4) (layer "B.Cu") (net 5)))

